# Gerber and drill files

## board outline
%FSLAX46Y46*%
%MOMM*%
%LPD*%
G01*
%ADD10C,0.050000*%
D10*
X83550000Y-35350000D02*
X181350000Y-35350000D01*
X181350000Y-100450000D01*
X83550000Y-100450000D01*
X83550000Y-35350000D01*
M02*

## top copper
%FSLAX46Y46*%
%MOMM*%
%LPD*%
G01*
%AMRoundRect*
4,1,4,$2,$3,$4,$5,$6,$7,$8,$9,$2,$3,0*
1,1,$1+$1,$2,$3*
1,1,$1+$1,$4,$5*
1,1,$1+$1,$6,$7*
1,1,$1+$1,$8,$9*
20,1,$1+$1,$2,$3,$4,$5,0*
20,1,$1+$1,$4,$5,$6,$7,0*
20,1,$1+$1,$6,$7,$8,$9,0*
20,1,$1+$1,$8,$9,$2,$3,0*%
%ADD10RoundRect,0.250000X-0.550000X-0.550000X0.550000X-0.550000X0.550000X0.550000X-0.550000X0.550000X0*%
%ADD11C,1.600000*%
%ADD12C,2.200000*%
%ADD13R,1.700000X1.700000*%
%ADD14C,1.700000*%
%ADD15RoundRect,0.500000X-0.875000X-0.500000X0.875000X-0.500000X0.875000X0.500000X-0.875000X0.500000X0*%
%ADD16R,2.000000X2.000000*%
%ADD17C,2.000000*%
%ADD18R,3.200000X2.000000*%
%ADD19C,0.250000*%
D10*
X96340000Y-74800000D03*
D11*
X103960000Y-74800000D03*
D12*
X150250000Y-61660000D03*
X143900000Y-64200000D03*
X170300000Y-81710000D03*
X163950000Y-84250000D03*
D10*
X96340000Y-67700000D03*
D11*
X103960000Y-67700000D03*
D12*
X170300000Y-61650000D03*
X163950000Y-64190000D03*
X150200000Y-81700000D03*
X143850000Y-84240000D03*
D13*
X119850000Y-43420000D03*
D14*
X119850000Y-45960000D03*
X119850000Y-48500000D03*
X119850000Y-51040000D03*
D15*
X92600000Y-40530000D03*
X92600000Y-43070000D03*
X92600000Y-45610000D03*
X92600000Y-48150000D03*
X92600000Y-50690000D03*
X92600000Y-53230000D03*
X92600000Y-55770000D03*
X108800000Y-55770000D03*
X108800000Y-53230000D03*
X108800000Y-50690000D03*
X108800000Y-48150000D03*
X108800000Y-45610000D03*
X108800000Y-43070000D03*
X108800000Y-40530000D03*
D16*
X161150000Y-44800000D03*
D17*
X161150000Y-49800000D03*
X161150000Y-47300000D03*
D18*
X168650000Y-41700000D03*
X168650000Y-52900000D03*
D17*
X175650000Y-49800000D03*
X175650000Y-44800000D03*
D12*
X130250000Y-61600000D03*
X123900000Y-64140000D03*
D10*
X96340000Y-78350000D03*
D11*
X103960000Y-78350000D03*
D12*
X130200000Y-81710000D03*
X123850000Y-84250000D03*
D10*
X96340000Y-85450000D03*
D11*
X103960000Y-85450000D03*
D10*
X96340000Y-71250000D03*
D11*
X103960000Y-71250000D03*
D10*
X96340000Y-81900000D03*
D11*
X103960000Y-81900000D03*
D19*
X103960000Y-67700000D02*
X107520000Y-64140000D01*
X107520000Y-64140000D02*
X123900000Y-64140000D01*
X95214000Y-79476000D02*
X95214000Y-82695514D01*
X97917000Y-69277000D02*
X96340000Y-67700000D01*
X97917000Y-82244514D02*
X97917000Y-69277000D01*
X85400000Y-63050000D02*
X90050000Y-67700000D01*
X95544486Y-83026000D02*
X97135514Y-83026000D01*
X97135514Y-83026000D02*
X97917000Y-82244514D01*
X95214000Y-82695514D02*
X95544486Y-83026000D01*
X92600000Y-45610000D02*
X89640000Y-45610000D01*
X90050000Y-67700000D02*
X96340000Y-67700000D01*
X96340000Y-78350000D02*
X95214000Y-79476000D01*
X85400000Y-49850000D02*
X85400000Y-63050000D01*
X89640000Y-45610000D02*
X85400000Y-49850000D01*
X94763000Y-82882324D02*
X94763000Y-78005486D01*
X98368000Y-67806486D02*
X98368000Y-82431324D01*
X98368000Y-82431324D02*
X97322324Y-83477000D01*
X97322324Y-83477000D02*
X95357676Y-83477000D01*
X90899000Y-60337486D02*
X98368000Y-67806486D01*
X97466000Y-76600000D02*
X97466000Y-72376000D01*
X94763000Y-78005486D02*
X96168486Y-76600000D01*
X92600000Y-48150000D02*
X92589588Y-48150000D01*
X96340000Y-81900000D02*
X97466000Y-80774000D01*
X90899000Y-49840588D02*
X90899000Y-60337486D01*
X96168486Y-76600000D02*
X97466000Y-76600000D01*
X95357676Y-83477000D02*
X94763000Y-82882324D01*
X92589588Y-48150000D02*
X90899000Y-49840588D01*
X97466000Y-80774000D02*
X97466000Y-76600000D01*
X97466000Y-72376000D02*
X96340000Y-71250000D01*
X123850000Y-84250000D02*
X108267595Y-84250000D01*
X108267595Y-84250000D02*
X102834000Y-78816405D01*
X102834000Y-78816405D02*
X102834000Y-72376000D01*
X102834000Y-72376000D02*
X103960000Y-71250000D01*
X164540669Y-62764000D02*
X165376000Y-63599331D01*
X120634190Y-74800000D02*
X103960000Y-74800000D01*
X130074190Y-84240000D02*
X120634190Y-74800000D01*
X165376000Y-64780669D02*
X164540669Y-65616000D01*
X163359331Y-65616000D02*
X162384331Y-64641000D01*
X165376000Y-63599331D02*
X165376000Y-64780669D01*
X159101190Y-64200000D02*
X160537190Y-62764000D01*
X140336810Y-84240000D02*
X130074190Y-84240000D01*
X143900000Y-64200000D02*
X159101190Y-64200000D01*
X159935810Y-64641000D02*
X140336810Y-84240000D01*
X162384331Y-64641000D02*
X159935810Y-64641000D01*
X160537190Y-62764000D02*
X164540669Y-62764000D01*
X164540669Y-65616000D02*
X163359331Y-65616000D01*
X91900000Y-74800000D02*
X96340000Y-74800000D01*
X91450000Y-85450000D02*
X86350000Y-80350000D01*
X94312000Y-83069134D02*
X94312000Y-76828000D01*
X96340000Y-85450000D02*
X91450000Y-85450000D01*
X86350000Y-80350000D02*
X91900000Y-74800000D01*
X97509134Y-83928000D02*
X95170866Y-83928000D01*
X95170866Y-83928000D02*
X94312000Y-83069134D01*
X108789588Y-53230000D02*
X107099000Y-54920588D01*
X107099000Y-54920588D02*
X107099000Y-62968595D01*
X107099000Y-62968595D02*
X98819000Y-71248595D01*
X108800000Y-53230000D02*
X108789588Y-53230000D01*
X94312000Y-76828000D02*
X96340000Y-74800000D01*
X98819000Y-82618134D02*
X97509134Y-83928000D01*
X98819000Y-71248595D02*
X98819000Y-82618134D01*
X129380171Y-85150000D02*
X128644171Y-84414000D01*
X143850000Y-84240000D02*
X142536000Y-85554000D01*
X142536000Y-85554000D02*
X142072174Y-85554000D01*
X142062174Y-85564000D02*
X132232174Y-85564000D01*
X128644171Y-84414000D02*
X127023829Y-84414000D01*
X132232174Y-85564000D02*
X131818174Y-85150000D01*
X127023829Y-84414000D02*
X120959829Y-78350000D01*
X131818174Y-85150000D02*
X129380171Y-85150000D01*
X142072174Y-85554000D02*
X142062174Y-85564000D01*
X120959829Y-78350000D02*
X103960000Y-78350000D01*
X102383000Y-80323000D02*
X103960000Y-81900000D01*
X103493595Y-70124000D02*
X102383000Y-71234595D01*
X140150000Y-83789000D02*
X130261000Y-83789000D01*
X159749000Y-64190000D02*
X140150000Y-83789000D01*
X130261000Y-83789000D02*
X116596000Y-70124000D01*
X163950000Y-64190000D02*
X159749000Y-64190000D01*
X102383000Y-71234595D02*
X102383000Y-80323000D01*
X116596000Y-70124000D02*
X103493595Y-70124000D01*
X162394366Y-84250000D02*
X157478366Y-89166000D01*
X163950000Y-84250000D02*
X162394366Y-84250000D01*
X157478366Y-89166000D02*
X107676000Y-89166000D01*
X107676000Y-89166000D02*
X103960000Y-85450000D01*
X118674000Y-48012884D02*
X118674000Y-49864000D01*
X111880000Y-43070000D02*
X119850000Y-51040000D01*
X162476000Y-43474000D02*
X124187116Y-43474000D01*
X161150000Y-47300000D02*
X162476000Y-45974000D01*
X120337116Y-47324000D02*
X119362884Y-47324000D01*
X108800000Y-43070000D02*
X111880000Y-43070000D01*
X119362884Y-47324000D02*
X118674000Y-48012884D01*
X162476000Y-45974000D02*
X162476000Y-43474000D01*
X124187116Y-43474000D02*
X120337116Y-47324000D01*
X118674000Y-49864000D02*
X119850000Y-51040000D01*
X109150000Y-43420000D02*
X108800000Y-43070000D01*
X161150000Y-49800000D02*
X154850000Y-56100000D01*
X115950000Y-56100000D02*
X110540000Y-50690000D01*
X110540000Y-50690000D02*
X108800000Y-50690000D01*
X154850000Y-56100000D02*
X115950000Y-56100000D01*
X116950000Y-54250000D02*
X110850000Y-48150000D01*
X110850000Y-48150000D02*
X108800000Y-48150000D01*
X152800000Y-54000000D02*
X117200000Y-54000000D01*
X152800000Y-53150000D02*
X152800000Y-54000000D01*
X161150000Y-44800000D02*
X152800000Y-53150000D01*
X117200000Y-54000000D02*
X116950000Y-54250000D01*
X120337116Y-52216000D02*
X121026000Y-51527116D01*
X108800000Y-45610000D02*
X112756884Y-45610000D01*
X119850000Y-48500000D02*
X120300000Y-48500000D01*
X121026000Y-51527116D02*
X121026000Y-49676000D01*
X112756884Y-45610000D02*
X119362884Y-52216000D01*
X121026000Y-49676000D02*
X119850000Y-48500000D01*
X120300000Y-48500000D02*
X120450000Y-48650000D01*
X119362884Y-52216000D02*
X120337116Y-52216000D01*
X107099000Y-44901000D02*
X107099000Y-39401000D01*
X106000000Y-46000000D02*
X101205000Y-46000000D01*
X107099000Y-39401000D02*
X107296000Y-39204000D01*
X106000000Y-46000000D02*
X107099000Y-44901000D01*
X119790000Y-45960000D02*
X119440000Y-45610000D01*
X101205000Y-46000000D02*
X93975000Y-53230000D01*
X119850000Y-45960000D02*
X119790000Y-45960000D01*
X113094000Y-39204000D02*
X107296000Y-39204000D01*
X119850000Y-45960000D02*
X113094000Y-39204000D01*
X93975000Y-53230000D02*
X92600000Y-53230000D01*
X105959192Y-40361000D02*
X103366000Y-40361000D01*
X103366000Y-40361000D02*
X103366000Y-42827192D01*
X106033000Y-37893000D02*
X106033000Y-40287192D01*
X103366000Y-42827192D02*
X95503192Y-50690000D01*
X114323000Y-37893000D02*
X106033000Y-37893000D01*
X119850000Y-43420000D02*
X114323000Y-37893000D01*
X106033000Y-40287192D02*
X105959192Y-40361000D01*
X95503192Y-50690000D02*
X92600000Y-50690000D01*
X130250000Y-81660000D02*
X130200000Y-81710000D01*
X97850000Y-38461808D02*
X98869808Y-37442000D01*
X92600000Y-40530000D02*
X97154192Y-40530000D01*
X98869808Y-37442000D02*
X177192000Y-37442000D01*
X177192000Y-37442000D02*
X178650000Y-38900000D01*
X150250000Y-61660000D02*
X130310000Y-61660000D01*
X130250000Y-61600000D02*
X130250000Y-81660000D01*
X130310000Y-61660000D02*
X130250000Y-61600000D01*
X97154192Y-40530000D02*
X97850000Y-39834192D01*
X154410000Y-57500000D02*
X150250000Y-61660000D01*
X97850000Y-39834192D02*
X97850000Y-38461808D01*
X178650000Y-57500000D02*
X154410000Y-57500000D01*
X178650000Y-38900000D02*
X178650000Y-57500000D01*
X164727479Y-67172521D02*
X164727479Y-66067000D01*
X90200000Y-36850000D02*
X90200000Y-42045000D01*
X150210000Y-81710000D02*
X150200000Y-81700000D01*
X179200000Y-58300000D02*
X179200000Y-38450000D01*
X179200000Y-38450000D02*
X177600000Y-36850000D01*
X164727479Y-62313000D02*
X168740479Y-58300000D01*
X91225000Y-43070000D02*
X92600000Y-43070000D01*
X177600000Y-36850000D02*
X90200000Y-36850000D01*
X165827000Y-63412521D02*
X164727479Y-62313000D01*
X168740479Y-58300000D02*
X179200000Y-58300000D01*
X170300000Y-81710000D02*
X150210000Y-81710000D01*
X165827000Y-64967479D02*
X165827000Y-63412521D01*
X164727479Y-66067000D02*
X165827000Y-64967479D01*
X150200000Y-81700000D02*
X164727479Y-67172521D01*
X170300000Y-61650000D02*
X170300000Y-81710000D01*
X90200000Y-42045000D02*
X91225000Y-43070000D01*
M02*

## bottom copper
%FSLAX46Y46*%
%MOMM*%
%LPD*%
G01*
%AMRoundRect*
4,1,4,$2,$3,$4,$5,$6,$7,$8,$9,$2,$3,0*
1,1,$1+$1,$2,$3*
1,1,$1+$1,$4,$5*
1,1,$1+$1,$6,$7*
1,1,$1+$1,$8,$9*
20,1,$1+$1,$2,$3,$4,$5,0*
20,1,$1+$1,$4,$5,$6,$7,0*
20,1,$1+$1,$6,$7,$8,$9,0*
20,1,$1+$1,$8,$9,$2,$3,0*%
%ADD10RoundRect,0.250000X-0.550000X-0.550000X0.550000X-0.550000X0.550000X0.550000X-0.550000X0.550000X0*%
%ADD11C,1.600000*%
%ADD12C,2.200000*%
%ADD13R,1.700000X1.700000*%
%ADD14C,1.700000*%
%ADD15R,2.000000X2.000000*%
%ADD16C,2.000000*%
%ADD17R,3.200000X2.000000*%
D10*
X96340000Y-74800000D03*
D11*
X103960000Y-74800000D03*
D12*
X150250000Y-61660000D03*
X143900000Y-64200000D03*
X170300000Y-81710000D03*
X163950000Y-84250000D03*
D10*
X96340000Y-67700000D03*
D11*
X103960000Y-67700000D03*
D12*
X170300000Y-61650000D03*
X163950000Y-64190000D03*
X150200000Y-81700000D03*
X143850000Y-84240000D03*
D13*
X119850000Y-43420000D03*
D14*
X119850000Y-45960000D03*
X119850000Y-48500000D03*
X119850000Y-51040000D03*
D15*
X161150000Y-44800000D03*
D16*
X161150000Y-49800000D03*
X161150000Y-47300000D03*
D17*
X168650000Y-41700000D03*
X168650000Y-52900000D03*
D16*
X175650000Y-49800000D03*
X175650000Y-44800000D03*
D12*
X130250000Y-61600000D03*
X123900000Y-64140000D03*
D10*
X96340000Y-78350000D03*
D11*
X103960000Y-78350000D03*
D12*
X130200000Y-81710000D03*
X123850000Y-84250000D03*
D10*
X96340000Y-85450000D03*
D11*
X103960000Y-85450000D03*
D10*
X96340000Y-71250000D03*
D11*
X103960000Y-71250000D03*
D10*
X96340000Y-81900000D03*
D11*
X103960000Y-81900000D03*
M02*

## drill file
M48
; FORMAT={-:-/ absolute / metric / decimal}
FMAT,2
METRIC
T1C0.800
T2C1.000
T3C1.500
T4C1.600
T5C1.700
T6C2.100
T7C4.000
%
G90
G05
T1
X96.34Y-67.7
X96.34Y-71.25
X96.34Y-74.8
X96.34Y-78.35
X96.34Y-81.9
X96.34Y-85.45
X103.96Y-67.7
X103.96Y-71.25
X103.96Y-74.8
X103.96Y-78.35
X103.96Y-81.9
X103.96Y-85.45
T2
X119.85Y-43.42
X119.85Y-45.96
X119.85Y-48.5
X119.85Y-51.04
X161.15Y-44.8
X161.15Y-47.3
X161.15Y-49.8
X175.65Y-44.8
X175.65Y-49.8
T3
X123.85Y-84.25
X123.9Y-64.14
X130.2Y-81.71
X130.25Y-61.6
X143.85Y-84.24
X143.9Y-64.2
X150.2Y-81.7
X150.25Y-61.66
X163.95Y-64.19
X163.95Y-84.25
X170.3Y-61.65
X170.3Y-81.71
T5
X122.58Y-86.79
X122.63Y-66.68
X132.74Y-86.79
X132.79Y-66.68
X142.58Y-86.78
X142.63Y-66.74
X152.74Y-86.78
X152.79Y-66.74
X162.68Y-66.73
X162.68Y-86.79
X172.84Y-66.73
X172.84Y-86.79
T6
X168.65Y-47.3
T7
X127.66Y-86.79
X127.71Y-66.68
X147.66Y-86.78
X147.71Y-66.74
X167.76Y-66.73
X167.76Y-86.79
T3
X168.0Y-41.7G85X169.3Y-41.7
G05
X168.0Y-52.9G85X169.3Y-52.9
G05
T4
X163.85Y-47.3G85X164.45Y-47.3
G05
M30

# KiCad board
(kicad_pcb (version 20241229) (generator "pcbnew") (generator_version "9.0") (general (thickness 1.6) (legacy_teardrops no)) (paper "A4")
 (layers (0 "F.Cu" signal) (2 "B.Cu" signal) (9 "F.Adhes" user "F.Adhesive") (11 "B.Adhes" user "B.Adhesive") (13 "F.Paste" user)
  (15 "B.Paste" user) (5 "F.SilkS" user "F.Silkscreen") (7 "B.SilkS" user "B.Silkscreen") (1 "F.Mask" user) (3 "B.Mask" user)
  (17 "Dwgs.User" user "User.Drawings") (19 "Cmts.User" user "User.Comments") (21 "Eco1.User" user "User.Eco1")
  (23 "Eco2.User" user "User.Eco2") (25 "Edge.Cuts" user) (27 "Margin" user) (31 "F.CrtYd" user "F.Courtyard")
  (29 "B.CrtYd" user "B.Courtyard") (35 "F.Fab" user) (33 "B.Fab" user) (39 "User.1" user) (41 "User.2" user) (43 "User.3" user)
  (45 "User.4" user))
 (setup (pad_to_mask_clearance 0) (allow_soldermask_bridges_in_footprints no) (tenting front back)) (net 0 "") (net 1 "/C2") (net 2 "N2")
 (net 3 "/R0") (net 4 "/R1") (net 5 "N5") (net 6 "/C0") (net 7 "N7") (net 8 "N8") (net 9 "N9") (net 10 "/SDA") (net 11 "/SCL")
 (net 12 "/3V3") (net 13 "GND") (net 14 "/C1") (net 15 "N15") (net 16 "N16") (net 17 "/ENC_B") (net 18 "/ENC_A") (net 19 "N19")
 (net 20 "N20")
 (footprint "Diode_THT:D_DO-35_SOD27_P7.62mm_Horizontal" (layer "F.Cu") (at 96.34 74.8)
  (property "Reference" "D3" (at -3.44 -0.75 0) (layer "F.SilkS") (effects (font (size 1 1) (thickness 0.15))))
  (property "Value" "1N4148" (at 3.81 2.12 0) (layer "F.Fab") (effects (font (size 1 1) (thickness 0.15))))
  (pad "1" thru_hole roundrect (at 0 0) (size 1.6 1.6) (drill 0.8) (layers "*.Cu" "*.Mask") (remove_unused_layers no)
   (roundrect_rratio 0.15625) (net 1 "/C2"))
  (pad "2" thru_hole circle (at 7.62 0) (size 1.6 1.6) (drill 0.8) (layers "*.Cu" "*.Mask") (remove_unused_layers no) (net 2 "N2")))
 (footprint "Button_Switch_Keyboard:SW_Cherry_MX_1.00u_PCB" (layer "F.Cu") (at 150.25 61.66)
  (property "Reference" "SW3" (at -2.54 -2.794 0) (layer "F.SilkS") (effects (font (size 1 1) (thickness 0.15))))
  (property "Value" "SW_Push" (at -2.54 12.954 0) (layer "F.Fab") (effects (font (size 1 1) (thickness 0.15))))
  (pad "" np_thru_hole circle (at -7.62 5.08) (size 1.7 1.7) (drill 1.7) (layers "*.Cu" "*.Mask"))
  (pad "" np_thru_hole circle (at -2.54 5.08) (size 4 4) (drill 4) (layers "*.Cu" "*.Mask"))
  (pad "" np_thru_hole circle (at 2.54 5.08) (size 1.7 1.7) (drill 1.7) (layers "*.Cu" "*.Mask"))
  (pad "1" thru_hole circle (at 0 0) (size 2.2 2.2) (drill 1.5) (layers "*.Cu" "*.Mask") (remove_unused_layers no) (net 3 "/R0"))
  (pad "2" thru_hole circle (at -6.35 2.54) (size 2.2 2.2) (drill 1.5) (layers "*.Cu" "*.Mask") (remove_unused_layers no) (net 2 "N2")))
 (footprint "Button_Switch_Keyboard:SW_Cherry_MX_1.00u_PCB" (layer "F.Cu") (at 170.3 81.71)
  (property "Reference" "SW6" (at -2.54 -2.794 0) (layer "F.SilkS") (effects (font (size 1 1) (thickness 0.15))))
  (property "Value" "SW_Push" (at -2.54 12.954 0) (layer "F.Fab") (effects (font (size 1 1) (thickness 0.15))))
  (pad "" np_thru_hole circle (at -7.62 5.08) (size 1.7 1.7) (drill 1.7) (layers "*.Cu" "*.Mask"))
  (pad "" np_thru_hole circle (at -2.54 5.08) (size 4 4) (drill 4) (layers "*.Cu" "*.Mask"))
  (pad "" np_thru_hole circle (at 2.54 5.08) (size 1.7 1.7) (drill 1.7) (layers "*.Cu" "*.Mask"))
  (pad "1" thru_hole circle (at 0 0) (size 2.2 2.2) (drill 1.5) (layers "*.Cu" "*.Mask") (remove_unused_layers no) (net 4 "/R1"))
  (pad "2" thru_hole circle (at -6.35 2.54) (size 2.2 2.2) (drill 1.5) (layers "*.Cu" "*.Mask") (remove_unused_layers no) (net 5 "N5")))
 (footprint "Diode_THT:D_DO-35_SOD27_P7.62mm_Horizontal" (layer "F.Cu") (at 96.34 67.7)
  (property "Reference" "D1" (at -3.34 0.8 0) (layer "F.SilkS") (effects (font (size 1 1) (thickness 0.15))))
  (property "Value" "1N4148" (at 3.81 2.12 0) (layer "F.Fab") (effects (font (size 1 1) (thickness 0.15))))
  (pad "1" thru_hole roundrect (at 0 0) (size 1.6 1.6) (drill 0.8) (layers "*.Cu" "*.Mask") (remove_unused_layers no)
   (roundrect_rratio 0.15625) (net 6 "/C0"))
  (pad "2" thru_hole circle (at 7.62 0) (size 1.6 1.6) (drill 0.8) (layers "*.Cu" "*.Mask") (remove_unused_layers no) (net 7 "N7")))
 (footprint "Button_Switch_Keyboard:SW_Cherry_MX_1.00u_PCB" (layer "F.Cu") (at 170.3 61.65)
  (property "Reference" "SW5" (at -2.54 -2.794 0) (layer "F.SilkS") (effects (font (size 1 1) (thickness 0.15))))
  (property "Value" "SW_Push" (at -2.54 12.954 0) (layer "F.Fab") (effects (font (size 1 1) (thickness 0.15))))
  (pad "" np_thru_hole circle (at -7.62 5.08) (size 1.7 1.7) (drill 1.7) (layers "*.Cu" "*.Mask"))
  (pad "" np_thru_hole circle (at -2.54 5.08) (size 4 4) (drill 4) (layers "*.Cu" "*.Mask"))
  (pad "" np_thru_hole circle (at 2.54 5.08) (size 1.7 1.7) (drill 1.7) (layers "*.Cu" "*.Mask"))
  (pad "1" thru_hole circle (at 0 0) (size 2.2 2.2) (drill 1.5) (layers "*.Cu" "*.Mask") (remove_unused_layers no) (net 4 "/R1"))
  (pad "2" thru_hole circle (at -6.35 2.54) (size 2.2 2.2) (drill 1.5) (layers "*.Cu" "*.Mask") (remove_unused_layers no) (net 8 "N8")))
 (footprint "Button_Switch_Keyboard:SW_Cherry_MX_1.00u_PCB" (layer "F.Cu") (at 150.2 81.7)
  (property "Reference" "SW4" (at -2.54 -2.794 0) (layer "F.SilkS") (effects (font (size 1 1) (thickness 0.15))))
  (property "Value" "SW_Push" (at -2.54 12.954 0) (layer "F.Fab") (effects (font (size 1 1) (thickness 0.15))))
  (pad "" np_thru_hole circle (at -7.62 5.08) (size 1.7 1.7) (drill 1.7) (layers "*.Cu" "*.Mask"))
  (pad "" np_thru_hole circle (at -2.54 5.08) (size 4 4) (drill 4) (layers "*.Cu" "*.Mask"))
  (pad "" np_thru_hole circle (at 2.54 5.08) (size 1.7 1.7) (drill 1.7) (layers "*.Cu" "*.Mask"))
  (pad "1" thru_hole circle (at 0 0) (size 2.2 2.2) (drill 1.5) (layers "*.Cu" "*.Mask") (remove_unused_layers no) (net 4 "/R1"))
  (pad "2" thru_hole circle (at -6.35 2.54) (size 2.2 2.2) (drill 1.5) (layers "*.Cu" "*.Mask") (remove_unused_layers no) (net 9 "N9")))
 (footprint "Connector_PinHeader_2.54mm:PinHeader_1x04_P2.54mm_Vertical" (layer "F.Cu") (at 119.85 43.42)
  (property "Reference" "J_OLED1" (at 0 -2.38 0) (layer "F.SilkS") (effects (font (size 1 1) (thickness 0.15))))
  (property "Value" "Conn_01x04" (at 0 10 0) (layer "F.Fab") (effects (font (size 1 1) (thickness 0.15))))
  (pad "1" thru_hole rect (at 0 0) (size 1.7 1.7) (drill 1) (layers "*.Cu" "*.Mask") (remove_unused_layers no) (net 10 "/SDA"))
  (pad "2" thru_hole circle (at 0 2.54) (size 1.7 1.7) (drill 1) (layers "*.Cu" "*.Mask") (remove_unused_layers no) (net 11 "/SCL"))
  (pad "3" thru_hole circle (at 0 5.08) (size 1.7 1.7) (drill 1) (layers "*.Cu" "*.Mask") (remove_unused_layers no) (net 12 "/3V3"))
  (pad "4" thru_hole circle (at 0 7.62) (size 1.7 1.7) (drill 1) (layers "*.Cu" "*.Mask") (remove_unused_layers no) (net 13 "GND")))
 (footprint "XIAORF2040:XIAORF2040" (layer "F.Cu") (at 100.7 48.15)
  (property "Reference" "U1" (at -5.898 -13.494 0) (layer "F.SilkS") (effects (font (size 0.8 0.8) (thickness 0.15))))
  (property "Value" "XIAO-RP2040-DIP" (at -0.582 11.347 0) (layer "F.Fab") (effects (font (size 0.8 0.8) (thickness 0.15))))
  (pad "1" smd roundrect (at -8.1 -7.62) (size 2.75 2) (layers "F.Cu" "F.Mask" "F.Paste") (roundrect_rratio 0.25) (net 3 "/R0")
   (solder_mask_margin 0.102))
  (pad "2" smd roundrect (at -8.1 -5.08) (size 2.75 2) (layers "F.Cu" "F.Mask" "F.Paste") (roundrect_rratio 0.25) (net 4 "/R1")
   (solder_mask_margin 0.102))
  (pad "3" smd roundrect (at -8.1 -2.54) (size 2.75 2) (layers "F.Cu" "F.Mask" "F.Paste") (roundrect_rratio 0.25) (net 6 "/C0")
   (solder_mask_margin 0.102))
  (pad "4" smd roundrect (at -8.1 0) (size 2.75 2) (layers "F.Cu" "F.Mask" "F.Paste") (roundrect_rratio 0.25) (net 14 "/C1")
   (solder_mask_margin 0.102))
  (pad "5" smd roundrect (at -8.1 2.54) (size 2.75 2) (layers "F.Cu" "F.Mask" "F.Paste") (roundrect_rratio 0.25) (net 10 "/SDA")
   (solder_mask_margin 0.102))
  (pad "6" smd roundrect (at -8.1 5.08) (size 2.75 2) (layers "F.Cu" "F.Mask" "F.Paste") (roundrect_rratio 0.25) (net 11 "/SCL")
   (solder_mask_margin 0.102))
  (pad "7" smd roundrect (at -8.1 7.62) (size 2.75 2) (layers "F.Cu" "F.Mask" "F.Paste") (roundrect_rratio 0.25) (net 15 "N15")
   (solder_mask_margin 0.102))
  (pad "8" smd roundrect (at 8.1 7.62) (size 2.75 2) (layers "F.Cu" "F.Mask" "F.Paste") (roundrect_rratio 0.25) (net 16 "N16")
   (solder_mask_margin 0.102))
  (pad "9" smd roundrect (at 8.1 5.08) (size 2.75 2) (layers "F.Cu" "F.Mask" "F.Paste") (roundrect_rratio 0.25) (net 1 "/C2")
   (solder_mask_margin 0.102))
  (pad "10" smd roundrect (at 8.1 2.54) (size 2.75 2) (layers "F.Cu" "F.Mask" "F.Paste") (roundrect_rratio 0.25) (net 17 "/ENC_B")
   (solder_mask_margin 0.102))
  (pad "11" smd roundrect (at 8.1 0) (size 2.75 2) (layers "F.Cu" "F.Mask" "F.Paste") (roundrect_rratio 0.25) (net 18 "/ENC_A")
   (solder_mask_margin 0.102))
  (pad "12" smd roundrect (at 8.1 -2.54) (size 2.75 2) (layers "F.Cu" "F.Mask" "F.Paste") (roundrect_rratio 0.25) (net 12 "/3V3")
   (solder_mask_margin 0.102))
  (pad "13" smd roundrect (at 8.1 -5.08) (size 2.75 2) (layers "F.Cu" "F.Mask" "F.Paste") (roundrect_rratio 0.25) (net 13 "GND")
   (solder_mask_margin 0.102))
  (pad "14" smd roundrect (at 8.1 -7.62) (size 2.75 2) (layers "F.Cu" "F.Mask" "F.Paste") (roundrect_rratio 0.25) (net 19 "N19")
   (solder_mask_margin 0.102))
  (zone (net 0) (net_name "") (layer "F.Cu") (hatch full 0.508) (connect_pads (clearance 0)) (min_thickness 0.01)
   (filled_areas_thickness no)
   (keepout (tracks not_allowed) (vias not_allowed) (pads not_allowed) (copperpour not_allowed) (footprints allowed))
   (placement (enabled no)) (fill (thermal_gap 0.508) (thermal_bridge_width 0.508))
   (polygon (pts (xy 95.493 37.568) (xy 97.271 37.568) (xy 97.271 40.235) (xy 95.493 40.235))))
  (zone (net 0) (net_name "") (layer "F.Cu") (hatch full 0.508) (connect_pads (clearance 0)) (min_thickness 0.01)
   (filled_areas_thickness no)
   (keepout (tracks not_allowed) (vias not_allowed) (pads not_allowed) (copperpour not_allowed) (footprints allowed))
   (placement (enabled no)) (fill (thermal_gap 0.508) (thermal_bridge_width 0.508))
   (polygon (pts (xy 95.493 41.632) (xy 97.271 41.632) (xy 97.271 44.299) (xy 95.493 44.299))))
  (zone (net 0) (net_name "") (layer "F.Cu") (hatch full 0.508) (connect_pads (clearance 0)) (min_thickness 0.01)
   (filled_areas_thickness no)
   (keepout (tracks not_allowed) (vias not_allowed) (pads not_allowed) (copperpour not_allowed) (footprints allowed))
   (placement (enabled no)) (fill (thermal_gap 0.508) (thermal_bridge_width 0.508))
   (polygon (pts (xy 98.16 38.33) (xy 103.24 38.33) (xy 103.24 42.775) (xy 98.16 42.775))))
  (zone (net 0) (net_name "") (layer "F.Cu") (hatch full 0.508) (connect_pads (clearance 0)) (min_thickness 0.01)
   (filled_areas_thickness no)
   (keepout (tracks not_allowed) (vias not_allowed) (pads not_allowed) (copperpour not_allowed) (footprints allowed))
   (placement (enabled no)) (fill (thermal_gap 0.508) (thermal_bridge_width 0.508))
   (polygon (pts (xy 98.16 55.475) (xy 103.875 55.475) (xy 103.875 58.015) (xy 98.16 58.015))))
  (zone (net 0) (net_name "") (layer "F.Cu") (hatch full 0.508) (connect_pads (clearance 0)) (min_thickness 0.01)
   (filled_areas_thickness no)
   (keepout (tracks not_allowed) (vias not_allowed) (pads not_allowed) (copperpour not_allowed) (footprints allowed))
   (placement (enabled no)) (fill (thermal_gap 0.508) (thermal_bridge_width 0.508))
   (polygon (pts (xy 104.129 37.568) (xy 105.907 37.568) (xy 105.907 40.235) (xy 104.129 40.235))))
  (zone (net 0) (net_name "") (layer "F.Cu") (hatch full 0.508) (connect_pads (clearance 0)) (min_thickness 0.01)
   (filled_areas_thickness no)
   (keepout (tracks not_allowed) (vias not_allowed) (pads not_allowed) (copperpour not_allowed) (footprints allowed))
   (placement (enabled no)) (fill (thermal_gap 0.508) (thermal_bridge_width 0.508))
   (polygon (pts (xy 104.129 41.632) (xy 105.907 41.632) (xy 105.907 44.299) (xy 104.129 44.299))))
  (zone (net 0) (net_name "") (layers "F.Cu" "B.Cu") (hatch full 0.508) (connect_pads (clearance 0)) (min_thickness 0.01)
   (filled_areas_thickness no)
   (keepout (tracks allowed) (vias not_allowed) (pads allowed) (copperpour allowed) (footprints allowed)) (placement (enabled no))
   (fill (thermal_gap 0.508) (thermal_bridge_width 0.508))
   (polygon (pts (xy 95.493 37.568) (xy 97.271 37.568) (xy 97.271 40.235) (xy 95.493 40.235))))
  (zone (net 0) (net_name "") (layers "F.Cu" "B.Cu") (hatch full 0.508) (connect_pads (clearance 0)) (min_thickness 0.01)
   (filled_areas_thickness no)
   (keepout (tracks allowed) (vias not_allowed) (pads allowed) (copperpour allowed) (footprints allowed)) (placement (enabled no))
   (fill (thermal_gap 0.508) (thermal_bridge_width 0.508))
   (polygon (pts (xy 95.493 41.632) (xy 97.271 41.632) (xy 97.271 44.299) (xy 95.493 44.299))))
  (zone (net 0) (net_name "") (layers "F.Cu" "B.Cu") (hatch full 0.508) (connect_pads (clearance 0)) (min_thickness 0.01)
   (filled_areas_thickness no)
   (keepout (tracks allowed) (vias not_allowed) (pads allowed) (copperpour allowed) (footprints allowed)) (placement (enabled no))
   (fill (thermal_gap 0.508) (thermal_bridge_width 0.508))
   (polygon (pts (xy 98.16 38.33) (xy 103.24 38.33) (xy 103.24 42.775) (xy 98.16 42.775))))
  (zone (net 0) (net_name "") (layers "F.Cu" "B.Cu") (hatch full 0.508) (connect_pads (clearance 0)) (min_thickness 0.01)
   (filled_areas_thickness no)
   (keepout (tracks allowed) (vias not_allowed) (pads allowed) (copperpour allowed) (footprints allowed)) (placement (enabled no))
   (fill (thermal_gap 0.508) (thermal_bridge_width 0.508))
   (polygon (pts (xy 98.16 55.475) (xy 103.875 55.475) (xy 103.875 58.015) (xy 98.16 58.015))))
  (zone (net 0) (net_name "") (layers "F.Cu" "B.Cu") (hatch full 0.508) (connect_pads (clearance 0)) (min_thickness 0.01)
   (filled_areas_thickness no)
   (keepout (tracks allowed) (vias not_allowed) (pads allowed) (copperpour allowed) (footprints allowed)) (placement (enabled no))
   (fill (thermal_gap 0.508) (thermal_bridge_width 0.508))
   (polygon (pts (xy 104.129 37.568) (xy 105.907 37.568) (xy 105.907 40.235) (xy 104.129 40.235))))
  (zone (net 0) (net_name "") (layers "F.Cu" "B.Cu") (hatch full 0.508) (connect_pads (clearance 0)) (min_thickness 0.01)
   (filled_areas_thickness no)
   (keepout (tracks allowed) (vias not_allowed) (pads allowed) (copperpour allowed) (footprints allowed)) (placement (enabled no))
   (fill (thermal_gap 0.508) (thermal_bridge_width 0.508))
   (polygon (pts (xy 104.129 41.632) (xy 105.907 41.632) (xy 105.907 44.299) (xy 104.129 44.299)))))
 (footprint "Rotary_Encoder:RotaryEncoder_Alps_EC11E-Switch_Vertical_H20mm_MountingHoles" (layer "F.Cu") (at 161.15 44.8)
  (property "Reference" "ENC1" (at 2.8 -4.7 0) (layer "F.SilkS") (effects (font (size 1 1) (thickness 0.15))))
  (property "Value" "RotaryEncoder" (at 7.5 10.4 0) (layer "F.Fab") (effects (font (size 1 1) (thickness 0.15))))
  (pad "" np_thru_hole oval (at 3 2.5) (size 2.2 1.6) (drill oval 2.2 1.6) (layers "*.Mask"))
  (pad "" np_thru_hole circle (at 7.5 2.5) (size 2.1 2.1) (drill 2.1) (layers "*.Mask"))
  (pad "A" thru_hole rect (at 0 0) (size 2 2) (drill 1) (layers "*.Cu" "*.Mask") (remove_unused_layers no) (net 18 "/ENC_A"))
  (pad "B" thru_hole circle (at 0 5) (size 2 2) (drill 1) (layers "*.Cu" "*.Mask") (remove_unused_layers no) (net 17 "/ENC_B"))
  (pad "C" thru_hole circle (at 0 2.5) (size 2 2) (drill 1) (layers "*.Cu" "*.Mask") (remove_unused_layers no) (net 13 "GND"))
  (pad "MP" thru_hole rect (at 7.5 -3.1) (size 3.2 2) (drill oval 2.8 1.5) (layers "*.Cu" "*.Mask") (remove_unused_layers no))
  (pad "MP" thru_hole rect (at 7.5 8.1) (size 3.2 2) (drill oval 2.8 1.5) (layers "*.Cu" "*.Mask") (remove_unused_layers no))
  (pad "S1" thru_hole circle (at 14.5 5) (size 2 2) (drill 1) (layers "*.Cu" "*.Mask") (remove_unused_layers no))
  (pad "S2" thru_hole circle (at 14.5 0) (size 2 2) (drill 1) (layers "*.Cu" "*.Mask") (remove_unused_layers no)))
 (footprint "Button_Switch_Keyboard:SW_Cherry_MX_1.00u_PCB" (layer "F.Cu") (at 130.25 61.6)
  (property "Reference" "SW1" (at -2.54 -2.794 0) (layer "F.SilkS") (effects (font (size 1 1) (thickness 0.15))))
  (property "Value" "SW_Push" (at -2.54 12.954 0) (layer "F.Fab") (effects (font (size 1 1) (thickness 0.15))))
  (pad "" np_thru_hole circle (at -7.62 5.08) (size 1.7 1.7) (drill 1.7) (layers "*.Cu" "*.Mask"))
  (pad "" np_thru_hole circle (at -2.54 5.08) (size 4 4) (drill 4) (layers "*.Cu" "*.Mask"))
  (pad "" np_thru_hole circle (at 2.54 5.08) (size 1.7 1.7) (drill 1.7) (layers "*.Cu" "*.Mask"))
  (pad "1" thru_hole circle (at 0 0) (size 2.2 2.2) (drill 1.5) (layers "*.Cu" "*.Mask") (remove_unused_layers no) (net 3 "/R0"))
  (pad "2" thru_hole circle (at -6.35 2.54) (size 2.2 2.2) (drill 1.5) (layers "*.Cu" "*.Mask") (remove_unused_layers no) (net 7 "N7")))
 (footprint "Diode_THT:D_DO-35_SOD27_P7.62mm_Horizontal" (layer "F.Cu") (at 96.34 78.35)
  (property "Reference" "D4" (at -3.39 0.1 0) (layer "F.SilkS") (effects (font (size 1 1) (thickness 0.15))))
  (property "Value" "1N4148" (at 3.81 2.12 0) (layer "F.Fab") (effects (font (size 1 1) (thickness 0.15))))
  (pad "1" thru_hole roundrect (at 0 0) (size 1.6 1.6) (drill 0.8) (layers "*.Cu" "*.Mask") (remove_unused_layers no)
   (roundrect_rratio 0.15625) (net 6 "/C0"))
  (pad "2" thru_hole circle (at 7.62 0) (size 1.6 1.6) (drill 0.8) (layers "*.Cu" "*.Mask") (remove_unused_layers no) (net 9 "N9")))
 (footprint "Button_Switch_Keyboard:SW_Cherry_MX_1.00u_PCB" (layer "F.Cu") (at 130.2 81.71)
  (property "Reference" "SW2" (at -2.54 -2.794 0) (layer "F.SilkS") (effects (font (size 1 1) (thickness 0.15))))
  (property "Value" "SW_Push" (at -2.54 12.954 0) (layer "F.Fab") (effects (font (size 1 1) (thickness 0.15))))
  (pad "" np_thru_hole circle (at -7.62 5.08) (size 1.7 1.7) (drill 1.7) (layers "*.Cu" "*.Mask"))
  (pad "" np_thru_hole circle (at -2.54 5.08) (size 4 4) (drill 4) (layers "*.Cu" "*.Mask"))
  (pad "" np_thru_hole circle (at 2.54 5.08) (size 1.7 1.7) (drill 1.7) (layers "*.Cu" "*.Mask"))
  (pad "1" thru_hole circle (at 0 0) (size 2.2 2.2) (drill 1.5) (layers "*.Cu" "*.Mask") (remove_unused_layers no) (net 3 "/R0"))
  (pad "2" thru_hole circle (at -6.35 2.54) (size 2.2 2.2) (drill 1.5) (layers "*.Cu" "*.Mask") (remove_unused_layers no) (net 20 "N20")))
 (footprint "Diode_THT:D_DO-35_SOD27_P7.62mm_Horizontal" (layer "F.Cu") (at 96.34 85.45)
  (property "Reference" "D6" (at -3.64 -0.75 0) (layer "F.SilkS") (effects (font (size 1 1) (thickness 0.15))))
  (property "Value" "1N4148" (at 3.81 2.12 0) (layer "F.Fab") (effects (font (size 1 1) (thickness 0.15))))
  (pad "1" thru_hole roundrect (at 0 0) (size 1.6 1.6) (drill 0.8) (layers "*.Cu" "*.Mask") (remove_unused_layers no)
   (roundrect_rratio 0.15625) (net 1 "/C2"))
  (pad "2" thru_hole circle (at 7.62 0) (size 1.6 1.6) (drill 0.8) (layers "*.Cu" "*.Mask") (remove_unused_layers no) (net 5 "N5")))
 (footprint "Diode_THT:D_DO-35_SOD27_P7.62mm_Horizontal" (layer "F.Cu") (at 96.34 71.25)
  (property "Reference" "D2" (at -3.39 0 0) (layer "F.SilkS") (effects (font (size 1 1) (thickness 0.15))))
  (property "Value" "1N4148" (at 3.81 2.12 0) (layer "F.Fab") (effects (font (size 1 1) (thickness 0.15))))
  (pad "1" thru_hole roundrect (at 0 0) (size 1.6 1.6) (drill 0.8) (layers "*.Cu" "*.Mask") (remove_unused_layers no)
   (roundrect_rratio 0.15625) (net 14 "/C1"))
  (pad "2" thru_hole circle (at 7.62 0) (size 1.6 1.6) (drill 0.8) (layers "*.Cu" "*.Mask") (remove_unused_layers no) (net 20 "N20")))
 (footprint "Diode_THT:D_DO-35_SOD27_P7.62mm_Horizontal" (layer "F.Cu") (at 96.34 81.9)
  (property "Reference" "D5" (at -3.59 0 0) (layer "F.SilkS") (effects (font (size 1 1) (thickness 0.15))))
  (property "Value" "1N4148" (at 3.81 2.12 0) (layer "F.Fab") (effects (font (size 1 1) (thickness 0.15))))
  (pad "1" thru_hole roundrect (at 0 0) (size 1.6 1.6) (drill 0.8) (layers "*.Cu" "*.Mask") (remove_unused_layers no)
   (roundrect_rratio 0.15625) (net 14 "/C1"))
  (pad "2" thru_hole circle (at 7.62 0) (size 1.6 1.6) (drill 0.8) (layers "*.Cu" "*.Mask") (remove_unused_layers no) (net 8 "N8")))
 (gr_rect (start 83.55 35.35) (end 181.35 100.45) (stroke (width 0.05) (type default)) (fill no) (layer "Edge.Cuts"))
 (segment (start 103.96 67.7) (end 107.52 64.14) (width 0.25) (layer "F.Cu") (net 7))
 (segment (start 107.52 64.14) (end 123.9 64.14) (width 0.25) (layer "F.Cu") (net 7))
 (segment (start 95.214 79.476) (end 95.214 82.695514) (width 0.25) (layer "F.Cu") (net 6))
 (segment (start 97.917 69.277) (end 96.34 67.7) (width 0.25) (layer "F.Cu") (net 6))
 (segment (start 97.917 82.244514) (end 97.917 69.277) (width 0.25) (layer "F.Cu") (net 6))
 (segment (start 85.4 63.05) (end 90.05 67.7) (width 0.25) (layer "F.Cu") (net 6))
 (segment (start 95.544486 83.026) (end 97.135514 83.026) (width 0.25) (layer "F.Cu") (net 6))
 (segment (start 97.135514 83.026) (end 97.917 82.244514) (width 0.25) (layer "F.Cu") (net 6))
 (segment (start 95.214 82.695514) (end 95.544486 83.026) (width 0.25) (layer "F.Cu") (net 6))
 (segment (start 92.6 45.61) (end 89.64 45.61) (width 0.25) (layer "F.Cu") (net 6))
 (segment (start 90.05 67.7) (end 96.34 67.7) (width 0.25) (layer "F.Cu") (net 6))
 (segment (start 96.34 78.35) (end 95.214 79.476) (width 0.25) (layer "F.Cu") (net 6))
 (segment (start 85.4 49.85) (end 85.4 63.05) (width 0.25) (layer "F.Cu") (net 6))
 (segment (start 89.64 45.61) (end 85.4 49.85) (width 0.25) (layer "F.Cu") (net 6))
 (segment (start 94.763 82.882324) (end 94.763 78.005486) (width 0.25) (layer "F.Cu") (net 14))
 (segment (start 98.368 67.806486) (end 98.368 82.431324) (width 0.25) (layer "F.Cu") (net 14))
 (segment (start 98.368 82.431324) (end 97.322324 83.477) (width 0.25) (layer "F.Cu") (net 14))
 (segment (start 97.322324 83.477) (end 95.357676 83.477) (width 0.25) (layer "F.Cu") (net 14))
 (segment (start 90.899 60.337486) (end 98.368 67.806486) (width 0.25) (layer "F.Cu") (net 14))
 (segment (start 97.466 76.6) (end 97.466 72.376) (width 0.25) (layer "F.Cu") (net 14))
 (segment (start 94.763 78.005486) (end 96.168486 76.6) (width 0.25) (layer "F.Cu") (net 14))
 (segment (start 92.6 48.15) (end 92.589588 48.15) (width 0.25) (layer "F.Cu") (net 14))
 (segment (start 96.34 81.9) (end 97.466 80.774) (width 0.25) (layer "F.Cu") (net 14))
 (segment (start 90.899 49.840588) (end 90.899 60.337486) (width 0.25) (layer "F.Cu") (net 14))
 (segment (start 96.168486 76.6) (end 97.466 76.6) (width 0.25) (layer "F.Cu") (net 14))
 (segment (start 95.357676 83.477) (end 94.763 82.882324) (width 0.25) (layer "F.Cu") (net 14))
 (segment (start 92.589588 48.15) (end 90.899 49.840588) (width 0.25) (layer "F.Cu") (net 14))
 (segment (start 97.466 80.774) (end 97.466 76.6) (width 0.25) (layer "F.Cu") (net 14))
 (segment (start 97.466 72.376) (end 96.34 71.25) (width 0.25) (layer "F.Cu") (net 14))
 (segment (start 123.85 84.25) (end 108.267595 84.25) (width 0.25) (layer "F.Cu") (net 20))
 (segment (start 108.267595 84.25) (end 102.834 78.816405) (width 0.25) (layer "F.Cu") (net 20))
 (segment (start 102.834 78.816405) (end 102.834 72.376) (width 0.25) (layer "F.Cu") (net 20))
 (segment (start 102.834 72.376) (end 103.96 71.25) (width 0.25) (layer "F.Cu") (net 20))
 (segment (start 164.540669 62.764) (end 165.376 63.599331) (width 0.25) (layer "F.Cu") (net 2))
 (segment (start 120.63419 74.8) (end 103.96 74.8) (width 0.25) (layer "F.Cu") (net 2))
 (segment (start 130.07419 84.24) (end 120.63419 74.8) (width 0.25) (layer "F.Cu") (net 2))
 (segment (start 165.376 64.780669) (end 164.540669 65.616) (width 0.25) (layer "F.Cu") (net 2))
 (segment (start 163.359331 65.616) (end 162.384331 64.641) (width 0.25) (layer "F.Cu") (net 2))
 (segment (start 165.376 63.599331) (end 165.376 64.780669) (width 0.25) (layer "F.Cu") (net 2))
 (segment (start 159.10119 64.2) (end 160.53719 62.764) (width 0.25) (layer "F.Cu") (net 2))
 (segment (start 140.33681 84.24) (end 130.07419 84.24) (width 0.25) (layer "F.Cu") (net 2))
 (segment (start 143.9 64.2) (end 159.10119 64.2) (width 0.25) (layer "F.Cu") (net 2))
 (segment (start 159.93581 64.641) (end 140.33681 84.24) (width 0.25) (layer "F.Cu") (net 2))
 (segment (start 162.384331 64.641) (end 159.93581 64.641) (width 0.25) (layer "F.Cu") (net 2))
 (segment (start 160.53719 62.764) (end 164.540669 62.764) (width 0.25) (layer "F.Cu") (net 2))
 (segment (start 164.540669 65.616) (end 163.359331 65.616) (width 0.25) (layer "F.Cu") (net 2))
 (segment (start 91.9 74.8) (end 96.34 74.8) (width 0.25) (layer "F.Cu") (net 1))
 (segment (start 91.45 85.45) (end 86.35 80.35) (width 0.25) (layer "F.Cu") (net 1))
 (segment (start 94.312 83.069134) (end 94.312 76.828) (width 0.25) (layer "F.Cu") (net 1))
 (segment (start 96.34 85.45) (end 91.45 85.45) (width 0.25) (layer "F.Cu") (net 1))
 (segment (start 86.35 80.35) (end 91.9 74.8) (width 0.25) (layer "F.Cu") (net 1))
 (segment (start 97.509134 83.928) (end 95.170866 83.928) (width 0.25) (layer "F.Cu") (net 1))
 (segment (start 95.170866 83.928) (end 94.312 83.069134) (width 0.25) (layer "F.Cu") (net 1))
 (segment (start 108.789588 53.23) (end 107.099 54.920588) (width 0.25) (layer "F.Cu") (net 1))
 (segment (start 107.099 54.920588) (end 107.099 62.968595) (width 0.25) (layer "F.Cu") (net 1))
 (segment (start 107.099 62.968595) (end 98.819 71.248595) (width 0.25) (layer "F.Cu") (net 1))
 (segment (start 108.8 53.23) (end 108.789588 53.23) (width 0.25) (layer "F.Cu") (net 1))
 (segment (start 94.312 76.828) (end 96.34 74.8) (width 0.25) (layer "F.Cu") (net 1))
 (segment (start 98.819 82.618134) (end 97.509134 83.928) (width 0.25) (layer "F.Cu") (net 1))
 (segment (start 98.819 71.248595) (end 98.819 82.618134) (width 0.25) (layer "F.Cu") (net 1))
 (segment (start 129.380171 85.15) (end 128.644171 84.414) (width 0.25) (layer "F.Cu") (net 9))
 (segment (start 143.85 84.24) (end 142.536 85.554) (width 0.25) (layer "F.Cu") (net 9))
 (segment (start 142.536 85.554) (end 142.072174 85.554) (width 0.25) (layer "F.Cu") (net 9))
 (segment (start 142.062174 85.564) (end 132.232174 85.564) (width 0.25) (layer "F.Cu") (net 9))
 (segment (start 128.644171 84.414) (end 127.023829 84.414) (width 0.25) (layer "F.Cu") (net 9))
 (segment (start 132.232174 85.564) (end 131.818174 85.15) (width 0.25) (layer "F.Cu") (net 9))
 (segment (start 127.023829 84.414) (end 120.959829 78.35) (width 0.25) (layer "F.Cu") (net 9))
 (segment (start 131.818174 85.15) (end 129.380171 85.15) (width 0.25) (layer "F.Cu") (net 9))
 (segment (start 142.072174 85.554) (end 142.062174 85.564) (width 0.25) (layer "F.Cu") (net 9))
 (segment (start 120.959829 78.35) (end 103.96 78.35) (width 0.25) (layer "F.Cu") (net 9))
 (segment (start 102.383 80.323) (end 103.96 81.9) (width 0.25) (layer "F.Cu") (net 8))
 (segment (start 103.493595 70.124) (end 102.383 71.234595) (width 0.25) (layer "F.Cu") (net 8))
 (segment (start 140.15 83.789) (end 130.261 83.789) (width 0.25) (layer "F.Cu") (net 8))
 (segment (start 159.749 64.19) (end 140.15 83.789) (width 0.25) (layer "F.Cu") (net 8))
 (segment (start 130.261 83.789) (end 116.596 70.124) (width 0.25) (layer "F.Cu") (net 8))
 (segment (start 163.95 64.19) (end 159.749 64.19) (width 0.25) (layer "F.Cu") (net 8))
 (segment (start 102.383 71.234595) (end 102.383 80.323) (width 0.25) (layer "F.Cu") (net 8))
 (segment (start 116.596 70.124) (end 103.493595 70.124) (width 0.25) (layer "F.Cu") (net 8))
 (segment (start 162.394366 84.25) (end 157.478366 89.166) (width 0.25) (layer "F.Cu") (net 5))
 (segment (start 163.95 84.25) (end 162.394366 84.25) (width 0.25) (layer "F.Cu") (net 5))
 (segment (start 157.478366 89.166) (end 107.676 89.166) (width 0.25) (layer "F.Cu") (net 5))
 (segment (start 107.676 89.166) (end 103.96 85.45) (width 0.25) (layer "F.Cu") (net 5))
 (segment (start 118.674 48.012884) (end 118.674 49.864) (width 0.25) (layer "F.Cu") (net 13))
 (segment (start 111.88 43.07) (end 119.85 51.04) (width 0.25) (layer "F.Cu") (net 13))
 (segment (start 162.476 43.474) (end 124.187116 43.474) (width 0.25) (layer "F.Cu") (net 13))
 (segment (start 161.15 47.3) (end 162.476 45.974) (width 0.25) (layer "F.Cu") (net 13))
 (segment (start 120.337116 47.324) (end 119.362884 47.324) (width 0.25) (layer "F.Cu") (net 13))
 (segment (start 108.8 43.07) (end 111.88 43.07) (width 0.25) (layer "F.Cu") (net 13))
 (segment (start 119.362884 47.324) (end 118.674 48.012884) (width 0.25) (layer "F.Cu") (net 13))
 (segment (start 162.476 45.974) (end 162.476 43.474) (width 0.25) (layer "F.Cu") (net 13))
 (segment (start 124.187116 43.474) (end 120.337116 47.324) (width 0.25) (layer "F.Cu") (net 13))
 (segment (start 118.674 49.864) (end 119.85 51.04) (width 0.25) (layer "F.Cu") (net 13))
 (segment (start 109.15 43.42) (end 108.8 43.07) (width 0.25) (layer "F.Cu") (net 13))
 (segment (start 161.15 49.8) (end 154.85 56.1) (width 0.25) (layer "F.Cu") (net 17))
 (segment (start 115.95 56.1) (end 110.54 50.69) (width 0.25) (layer "F.Cu") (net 17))
 (segment (start 110.54 50.69) (end 108.8 50.69) (width 0.25) (layer "F.Cu") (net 17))
 (segment (start 154.85 56.1) (end 115.95 56.1) (width 0.25) (layer "F.Cu") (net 17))
 (segment (start 116.95 54.25) (end 110.85 48.15) (width 0.25) (layer "F.Cu") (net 18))
 (segment (start 110.85 48.15) (end 108.8 48.15) (width 0.25) (layer "F.Cu") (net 18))
 (segment (start 152.8 54) (end 117.2 54) (width 0.25) (layer "F.Cu") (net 18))
 (segment (start 152.8 53.15) (end 152.8 54) (width 0.25) (layer "F.Cu") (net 18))
 (segment (start 161.15 44.8) (end 152.8 53.15) (width 0.25) (layer "F.Cu") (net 18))
 (segment (start 117.2 54) (end 116.95 54.25) (width 0.25) (layer "F.Cu") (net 18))
 (segment (start 120.337116 52.216) (end 121.026 51.527116) (width 0.25) (layer "F.Cu") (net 12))
 (segment (start 108.8 45.61) (end 112.756884 45.61) (width 0.25) (layer "F.Cu") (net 12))
 (segment (start 119.85 48.5) (end 120.3 48.5) (width 0.25) (layer "F.Cu") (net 12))
 (segment (start 121.026 51.527116) (end 121.026 49.676) (width 0.25) (layer "F.Cu") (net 12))
 (segment (start 112.756884 45.61) (end 119.362884 52.216) (width 0.25) (layer "F.Cu") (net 12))
 (segment (start 121.026 49.676) (end 119.85 48.5) (width 0.25) (layer "F.Cu") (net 12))
 (segment (start 120.3 48.5) (end 120.45 48.65) (width 0.25) (layer "F.Cu") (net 12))
 (segment (start 119.362884 52.216) (end 120.337116 52.216) (width 0.25) (layer "F.Cu") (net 12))
 (segment (start 107.099 44.901) (end 107.099 39.401) (width 0.25) (layer "F.Cu") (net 11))
 (segment (start 106 46) (end 101.205 46) (width 0.25) (layer "F.Cu") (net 11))
 (segment (start 107.099 39.401) (end 107.296 39.204) (width 0.25) (layer "F.Cu") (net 11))
 (segment (start 106 46) (end 107.099 44.901) (width 0.25) (layer "F.Cu") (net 11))
 (segment (start 119.79 45.96) (end 119.44 45.61) (width 0.25) (layer "F.Cu") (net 11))
 (segment (start 101.205 46) (end 93.975 53.23) (width 0.25) (layer "F.Cu") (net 11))
 (segment (start 119.85 45.96) (end 119.79 45.96) (width 0.25) (layer "F.Cu") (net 11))
 (segment (start 113.094 39.204) (end 107.296 39.204) (width 0.25) (layer "F.Cu") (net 11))
 (segment (start 119.85 45.96) (end 113.094 39.204) (width 0.25) (layer "F.Cu") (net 11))
 (segment (start 93.975 53.23) (end 92.6 53.23) (width 0.25) (layer "F.Cu") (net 11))
 (segment (start 105.959192 40.361) (end 103.366 40.361) (width 0.25) (layer "F.Cu") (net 10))
 (segment (start 103.366 40.361) (end 103.366 42.827192) (width 0.25) (layer "F.Cu") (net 10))
 (segment (start 106.033 37.893) (end 106.033 40.287192) (width 0.25) (layer "F.Cu") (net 10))
 (segment (start 103.366 42.827192) (end 95.503192 50.69) (width 0.25) (layer "F.Cu") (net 10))
 (segment (start 114.323 37.893) (end 106.033 37.893) (width 0.25) (layer "F.Cu") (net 10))
 (segment (start 119.85 43.42) (end 114.323 37.893) (width 0.25) (layer "F.Cu") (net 10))
 (segment (start 106.033 40.287192) (end 105.959192 40.361) (width 0.25) (layer "F.Cu") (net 10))
 (segment (start 95.503192 50.69) (end 92.6 50.69) (width 0.25) (layer "F.Cu") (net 10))
 (segment (start 130.25 81.66) (end 130.2 81.71) (width 0.25) (layer "F.Cu") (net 3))
 (segment (start 97.85 38.461808) (end 98.869808 37.442) (width 0.25) (layer "F.Cu") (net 3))
 (segment (start 92.6 40.53) (end 97.154192 40.53) (width 0.25) (layer "F.Cu") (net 3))
 (segment (start 98.869808 37.442) (end 177.192 37.442) (width 0.25) (layer "F.Cu") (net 3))
 (segment (start 177.192 37.442) (end 178.65 38.9) (width 0.25) (layer "F.Cu") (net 3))
 (segment (start 150.25 61.66) (end 130.31 61.66) (width 0.25) (layer "F.Cu") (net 3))
 (segment (start 130.25 61.6) (end 130.25 81.66) (width 0.25) (layer "F.Cu") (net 3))
 (segment (start 130.31 61.66) (end 130.25 61.6) (width 0.25) (layer "F.Cu") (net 3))
 (segment (start 97.154192 40.53) (end 97.85 39.834192) (width 0.25) (layer "F.Cu") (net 3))
 (segment (start 154.41 57.5) (end 150.25 61.66) (width 0.25) (layer "F.Cu") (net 3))
 (segment (start 97.85 39.834192) (end 97.85 38.461808) (width 0.25) (layer "F.Cu") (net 3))
 (segment (start 178.65 57.5) (end 154.41 57.5) (width 0.25) (layer "F.Cu") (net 3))
 (segment (start 178.65 38.9) (end 178.65 57.5) (width 0.25) (layer "F.Cu") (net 3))
 (segment (start 164.727479 67.172521) (end 164.727479 66.067) (width 0.25) (layer "F.Cu") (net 4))
 (segment (start 90.2 36.85) (end 90.2 42.045) (width 0.25) (layer "F.Cu") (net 4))
 (segment (start 150.21 81.71) (end 150.2 81.7) (width 0.25) (layer "F.Cu") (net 4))
 (segment (start 179.2 58.3) (end 179.2 38.45) (width 0.25) (layer "F.Cu") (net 4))
 (segment (start 179.2 38.45) (end 177.6 36.85) (width 0.25) (layer "F.Cu") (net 4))
 (segment (start 164.727479 62.313) (end 168.740479 58.3) (width 0.25) (layer "F.Cu") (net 4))
 (segment (start 91.225 43.07) (end 92.6 43.07) (width 0.25) (layer "F.Cu") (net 4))
 (segment (start 177.6 36.85) (end 90.2 36.85) (width 0.25) (layer "F.Cu") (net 4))
 (segment (start 165.827 63.412521) (end 164.727479 62.313) (width 0.25) (layer "F.Cu") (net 4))
 (segment (start 168.740479 58.3) (end 179.2 58.3) (width 0.25) (layer "F.Cu") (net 4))
 (segment (start 170.3 81.71) (end 150.21 81.71) (width 0.25) (layer "F.Cu") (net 4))
 (segment (start 165.827 64.967479) (end 165.827 63.412521) (width 0.25) (layer "F.Cu") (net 4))
 (segment (start 164.727479 66.067) (end 165.827 64.967479) (width 0.25) (layer "F.Cu") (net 4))
 (segment (start 150.2 81.7) (end 164.727479 67.172521) (width 0.25) (layer "F.Cu") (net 4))
 (segment (start 170.3 61.65) (end 170.3 81.71) (width 0.25) (layer "F.Cu") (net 4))
 (segment (start 90.2 42.045) (end 91.225 43.07) (width 0.25) (layer "F.Cu") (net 4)))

